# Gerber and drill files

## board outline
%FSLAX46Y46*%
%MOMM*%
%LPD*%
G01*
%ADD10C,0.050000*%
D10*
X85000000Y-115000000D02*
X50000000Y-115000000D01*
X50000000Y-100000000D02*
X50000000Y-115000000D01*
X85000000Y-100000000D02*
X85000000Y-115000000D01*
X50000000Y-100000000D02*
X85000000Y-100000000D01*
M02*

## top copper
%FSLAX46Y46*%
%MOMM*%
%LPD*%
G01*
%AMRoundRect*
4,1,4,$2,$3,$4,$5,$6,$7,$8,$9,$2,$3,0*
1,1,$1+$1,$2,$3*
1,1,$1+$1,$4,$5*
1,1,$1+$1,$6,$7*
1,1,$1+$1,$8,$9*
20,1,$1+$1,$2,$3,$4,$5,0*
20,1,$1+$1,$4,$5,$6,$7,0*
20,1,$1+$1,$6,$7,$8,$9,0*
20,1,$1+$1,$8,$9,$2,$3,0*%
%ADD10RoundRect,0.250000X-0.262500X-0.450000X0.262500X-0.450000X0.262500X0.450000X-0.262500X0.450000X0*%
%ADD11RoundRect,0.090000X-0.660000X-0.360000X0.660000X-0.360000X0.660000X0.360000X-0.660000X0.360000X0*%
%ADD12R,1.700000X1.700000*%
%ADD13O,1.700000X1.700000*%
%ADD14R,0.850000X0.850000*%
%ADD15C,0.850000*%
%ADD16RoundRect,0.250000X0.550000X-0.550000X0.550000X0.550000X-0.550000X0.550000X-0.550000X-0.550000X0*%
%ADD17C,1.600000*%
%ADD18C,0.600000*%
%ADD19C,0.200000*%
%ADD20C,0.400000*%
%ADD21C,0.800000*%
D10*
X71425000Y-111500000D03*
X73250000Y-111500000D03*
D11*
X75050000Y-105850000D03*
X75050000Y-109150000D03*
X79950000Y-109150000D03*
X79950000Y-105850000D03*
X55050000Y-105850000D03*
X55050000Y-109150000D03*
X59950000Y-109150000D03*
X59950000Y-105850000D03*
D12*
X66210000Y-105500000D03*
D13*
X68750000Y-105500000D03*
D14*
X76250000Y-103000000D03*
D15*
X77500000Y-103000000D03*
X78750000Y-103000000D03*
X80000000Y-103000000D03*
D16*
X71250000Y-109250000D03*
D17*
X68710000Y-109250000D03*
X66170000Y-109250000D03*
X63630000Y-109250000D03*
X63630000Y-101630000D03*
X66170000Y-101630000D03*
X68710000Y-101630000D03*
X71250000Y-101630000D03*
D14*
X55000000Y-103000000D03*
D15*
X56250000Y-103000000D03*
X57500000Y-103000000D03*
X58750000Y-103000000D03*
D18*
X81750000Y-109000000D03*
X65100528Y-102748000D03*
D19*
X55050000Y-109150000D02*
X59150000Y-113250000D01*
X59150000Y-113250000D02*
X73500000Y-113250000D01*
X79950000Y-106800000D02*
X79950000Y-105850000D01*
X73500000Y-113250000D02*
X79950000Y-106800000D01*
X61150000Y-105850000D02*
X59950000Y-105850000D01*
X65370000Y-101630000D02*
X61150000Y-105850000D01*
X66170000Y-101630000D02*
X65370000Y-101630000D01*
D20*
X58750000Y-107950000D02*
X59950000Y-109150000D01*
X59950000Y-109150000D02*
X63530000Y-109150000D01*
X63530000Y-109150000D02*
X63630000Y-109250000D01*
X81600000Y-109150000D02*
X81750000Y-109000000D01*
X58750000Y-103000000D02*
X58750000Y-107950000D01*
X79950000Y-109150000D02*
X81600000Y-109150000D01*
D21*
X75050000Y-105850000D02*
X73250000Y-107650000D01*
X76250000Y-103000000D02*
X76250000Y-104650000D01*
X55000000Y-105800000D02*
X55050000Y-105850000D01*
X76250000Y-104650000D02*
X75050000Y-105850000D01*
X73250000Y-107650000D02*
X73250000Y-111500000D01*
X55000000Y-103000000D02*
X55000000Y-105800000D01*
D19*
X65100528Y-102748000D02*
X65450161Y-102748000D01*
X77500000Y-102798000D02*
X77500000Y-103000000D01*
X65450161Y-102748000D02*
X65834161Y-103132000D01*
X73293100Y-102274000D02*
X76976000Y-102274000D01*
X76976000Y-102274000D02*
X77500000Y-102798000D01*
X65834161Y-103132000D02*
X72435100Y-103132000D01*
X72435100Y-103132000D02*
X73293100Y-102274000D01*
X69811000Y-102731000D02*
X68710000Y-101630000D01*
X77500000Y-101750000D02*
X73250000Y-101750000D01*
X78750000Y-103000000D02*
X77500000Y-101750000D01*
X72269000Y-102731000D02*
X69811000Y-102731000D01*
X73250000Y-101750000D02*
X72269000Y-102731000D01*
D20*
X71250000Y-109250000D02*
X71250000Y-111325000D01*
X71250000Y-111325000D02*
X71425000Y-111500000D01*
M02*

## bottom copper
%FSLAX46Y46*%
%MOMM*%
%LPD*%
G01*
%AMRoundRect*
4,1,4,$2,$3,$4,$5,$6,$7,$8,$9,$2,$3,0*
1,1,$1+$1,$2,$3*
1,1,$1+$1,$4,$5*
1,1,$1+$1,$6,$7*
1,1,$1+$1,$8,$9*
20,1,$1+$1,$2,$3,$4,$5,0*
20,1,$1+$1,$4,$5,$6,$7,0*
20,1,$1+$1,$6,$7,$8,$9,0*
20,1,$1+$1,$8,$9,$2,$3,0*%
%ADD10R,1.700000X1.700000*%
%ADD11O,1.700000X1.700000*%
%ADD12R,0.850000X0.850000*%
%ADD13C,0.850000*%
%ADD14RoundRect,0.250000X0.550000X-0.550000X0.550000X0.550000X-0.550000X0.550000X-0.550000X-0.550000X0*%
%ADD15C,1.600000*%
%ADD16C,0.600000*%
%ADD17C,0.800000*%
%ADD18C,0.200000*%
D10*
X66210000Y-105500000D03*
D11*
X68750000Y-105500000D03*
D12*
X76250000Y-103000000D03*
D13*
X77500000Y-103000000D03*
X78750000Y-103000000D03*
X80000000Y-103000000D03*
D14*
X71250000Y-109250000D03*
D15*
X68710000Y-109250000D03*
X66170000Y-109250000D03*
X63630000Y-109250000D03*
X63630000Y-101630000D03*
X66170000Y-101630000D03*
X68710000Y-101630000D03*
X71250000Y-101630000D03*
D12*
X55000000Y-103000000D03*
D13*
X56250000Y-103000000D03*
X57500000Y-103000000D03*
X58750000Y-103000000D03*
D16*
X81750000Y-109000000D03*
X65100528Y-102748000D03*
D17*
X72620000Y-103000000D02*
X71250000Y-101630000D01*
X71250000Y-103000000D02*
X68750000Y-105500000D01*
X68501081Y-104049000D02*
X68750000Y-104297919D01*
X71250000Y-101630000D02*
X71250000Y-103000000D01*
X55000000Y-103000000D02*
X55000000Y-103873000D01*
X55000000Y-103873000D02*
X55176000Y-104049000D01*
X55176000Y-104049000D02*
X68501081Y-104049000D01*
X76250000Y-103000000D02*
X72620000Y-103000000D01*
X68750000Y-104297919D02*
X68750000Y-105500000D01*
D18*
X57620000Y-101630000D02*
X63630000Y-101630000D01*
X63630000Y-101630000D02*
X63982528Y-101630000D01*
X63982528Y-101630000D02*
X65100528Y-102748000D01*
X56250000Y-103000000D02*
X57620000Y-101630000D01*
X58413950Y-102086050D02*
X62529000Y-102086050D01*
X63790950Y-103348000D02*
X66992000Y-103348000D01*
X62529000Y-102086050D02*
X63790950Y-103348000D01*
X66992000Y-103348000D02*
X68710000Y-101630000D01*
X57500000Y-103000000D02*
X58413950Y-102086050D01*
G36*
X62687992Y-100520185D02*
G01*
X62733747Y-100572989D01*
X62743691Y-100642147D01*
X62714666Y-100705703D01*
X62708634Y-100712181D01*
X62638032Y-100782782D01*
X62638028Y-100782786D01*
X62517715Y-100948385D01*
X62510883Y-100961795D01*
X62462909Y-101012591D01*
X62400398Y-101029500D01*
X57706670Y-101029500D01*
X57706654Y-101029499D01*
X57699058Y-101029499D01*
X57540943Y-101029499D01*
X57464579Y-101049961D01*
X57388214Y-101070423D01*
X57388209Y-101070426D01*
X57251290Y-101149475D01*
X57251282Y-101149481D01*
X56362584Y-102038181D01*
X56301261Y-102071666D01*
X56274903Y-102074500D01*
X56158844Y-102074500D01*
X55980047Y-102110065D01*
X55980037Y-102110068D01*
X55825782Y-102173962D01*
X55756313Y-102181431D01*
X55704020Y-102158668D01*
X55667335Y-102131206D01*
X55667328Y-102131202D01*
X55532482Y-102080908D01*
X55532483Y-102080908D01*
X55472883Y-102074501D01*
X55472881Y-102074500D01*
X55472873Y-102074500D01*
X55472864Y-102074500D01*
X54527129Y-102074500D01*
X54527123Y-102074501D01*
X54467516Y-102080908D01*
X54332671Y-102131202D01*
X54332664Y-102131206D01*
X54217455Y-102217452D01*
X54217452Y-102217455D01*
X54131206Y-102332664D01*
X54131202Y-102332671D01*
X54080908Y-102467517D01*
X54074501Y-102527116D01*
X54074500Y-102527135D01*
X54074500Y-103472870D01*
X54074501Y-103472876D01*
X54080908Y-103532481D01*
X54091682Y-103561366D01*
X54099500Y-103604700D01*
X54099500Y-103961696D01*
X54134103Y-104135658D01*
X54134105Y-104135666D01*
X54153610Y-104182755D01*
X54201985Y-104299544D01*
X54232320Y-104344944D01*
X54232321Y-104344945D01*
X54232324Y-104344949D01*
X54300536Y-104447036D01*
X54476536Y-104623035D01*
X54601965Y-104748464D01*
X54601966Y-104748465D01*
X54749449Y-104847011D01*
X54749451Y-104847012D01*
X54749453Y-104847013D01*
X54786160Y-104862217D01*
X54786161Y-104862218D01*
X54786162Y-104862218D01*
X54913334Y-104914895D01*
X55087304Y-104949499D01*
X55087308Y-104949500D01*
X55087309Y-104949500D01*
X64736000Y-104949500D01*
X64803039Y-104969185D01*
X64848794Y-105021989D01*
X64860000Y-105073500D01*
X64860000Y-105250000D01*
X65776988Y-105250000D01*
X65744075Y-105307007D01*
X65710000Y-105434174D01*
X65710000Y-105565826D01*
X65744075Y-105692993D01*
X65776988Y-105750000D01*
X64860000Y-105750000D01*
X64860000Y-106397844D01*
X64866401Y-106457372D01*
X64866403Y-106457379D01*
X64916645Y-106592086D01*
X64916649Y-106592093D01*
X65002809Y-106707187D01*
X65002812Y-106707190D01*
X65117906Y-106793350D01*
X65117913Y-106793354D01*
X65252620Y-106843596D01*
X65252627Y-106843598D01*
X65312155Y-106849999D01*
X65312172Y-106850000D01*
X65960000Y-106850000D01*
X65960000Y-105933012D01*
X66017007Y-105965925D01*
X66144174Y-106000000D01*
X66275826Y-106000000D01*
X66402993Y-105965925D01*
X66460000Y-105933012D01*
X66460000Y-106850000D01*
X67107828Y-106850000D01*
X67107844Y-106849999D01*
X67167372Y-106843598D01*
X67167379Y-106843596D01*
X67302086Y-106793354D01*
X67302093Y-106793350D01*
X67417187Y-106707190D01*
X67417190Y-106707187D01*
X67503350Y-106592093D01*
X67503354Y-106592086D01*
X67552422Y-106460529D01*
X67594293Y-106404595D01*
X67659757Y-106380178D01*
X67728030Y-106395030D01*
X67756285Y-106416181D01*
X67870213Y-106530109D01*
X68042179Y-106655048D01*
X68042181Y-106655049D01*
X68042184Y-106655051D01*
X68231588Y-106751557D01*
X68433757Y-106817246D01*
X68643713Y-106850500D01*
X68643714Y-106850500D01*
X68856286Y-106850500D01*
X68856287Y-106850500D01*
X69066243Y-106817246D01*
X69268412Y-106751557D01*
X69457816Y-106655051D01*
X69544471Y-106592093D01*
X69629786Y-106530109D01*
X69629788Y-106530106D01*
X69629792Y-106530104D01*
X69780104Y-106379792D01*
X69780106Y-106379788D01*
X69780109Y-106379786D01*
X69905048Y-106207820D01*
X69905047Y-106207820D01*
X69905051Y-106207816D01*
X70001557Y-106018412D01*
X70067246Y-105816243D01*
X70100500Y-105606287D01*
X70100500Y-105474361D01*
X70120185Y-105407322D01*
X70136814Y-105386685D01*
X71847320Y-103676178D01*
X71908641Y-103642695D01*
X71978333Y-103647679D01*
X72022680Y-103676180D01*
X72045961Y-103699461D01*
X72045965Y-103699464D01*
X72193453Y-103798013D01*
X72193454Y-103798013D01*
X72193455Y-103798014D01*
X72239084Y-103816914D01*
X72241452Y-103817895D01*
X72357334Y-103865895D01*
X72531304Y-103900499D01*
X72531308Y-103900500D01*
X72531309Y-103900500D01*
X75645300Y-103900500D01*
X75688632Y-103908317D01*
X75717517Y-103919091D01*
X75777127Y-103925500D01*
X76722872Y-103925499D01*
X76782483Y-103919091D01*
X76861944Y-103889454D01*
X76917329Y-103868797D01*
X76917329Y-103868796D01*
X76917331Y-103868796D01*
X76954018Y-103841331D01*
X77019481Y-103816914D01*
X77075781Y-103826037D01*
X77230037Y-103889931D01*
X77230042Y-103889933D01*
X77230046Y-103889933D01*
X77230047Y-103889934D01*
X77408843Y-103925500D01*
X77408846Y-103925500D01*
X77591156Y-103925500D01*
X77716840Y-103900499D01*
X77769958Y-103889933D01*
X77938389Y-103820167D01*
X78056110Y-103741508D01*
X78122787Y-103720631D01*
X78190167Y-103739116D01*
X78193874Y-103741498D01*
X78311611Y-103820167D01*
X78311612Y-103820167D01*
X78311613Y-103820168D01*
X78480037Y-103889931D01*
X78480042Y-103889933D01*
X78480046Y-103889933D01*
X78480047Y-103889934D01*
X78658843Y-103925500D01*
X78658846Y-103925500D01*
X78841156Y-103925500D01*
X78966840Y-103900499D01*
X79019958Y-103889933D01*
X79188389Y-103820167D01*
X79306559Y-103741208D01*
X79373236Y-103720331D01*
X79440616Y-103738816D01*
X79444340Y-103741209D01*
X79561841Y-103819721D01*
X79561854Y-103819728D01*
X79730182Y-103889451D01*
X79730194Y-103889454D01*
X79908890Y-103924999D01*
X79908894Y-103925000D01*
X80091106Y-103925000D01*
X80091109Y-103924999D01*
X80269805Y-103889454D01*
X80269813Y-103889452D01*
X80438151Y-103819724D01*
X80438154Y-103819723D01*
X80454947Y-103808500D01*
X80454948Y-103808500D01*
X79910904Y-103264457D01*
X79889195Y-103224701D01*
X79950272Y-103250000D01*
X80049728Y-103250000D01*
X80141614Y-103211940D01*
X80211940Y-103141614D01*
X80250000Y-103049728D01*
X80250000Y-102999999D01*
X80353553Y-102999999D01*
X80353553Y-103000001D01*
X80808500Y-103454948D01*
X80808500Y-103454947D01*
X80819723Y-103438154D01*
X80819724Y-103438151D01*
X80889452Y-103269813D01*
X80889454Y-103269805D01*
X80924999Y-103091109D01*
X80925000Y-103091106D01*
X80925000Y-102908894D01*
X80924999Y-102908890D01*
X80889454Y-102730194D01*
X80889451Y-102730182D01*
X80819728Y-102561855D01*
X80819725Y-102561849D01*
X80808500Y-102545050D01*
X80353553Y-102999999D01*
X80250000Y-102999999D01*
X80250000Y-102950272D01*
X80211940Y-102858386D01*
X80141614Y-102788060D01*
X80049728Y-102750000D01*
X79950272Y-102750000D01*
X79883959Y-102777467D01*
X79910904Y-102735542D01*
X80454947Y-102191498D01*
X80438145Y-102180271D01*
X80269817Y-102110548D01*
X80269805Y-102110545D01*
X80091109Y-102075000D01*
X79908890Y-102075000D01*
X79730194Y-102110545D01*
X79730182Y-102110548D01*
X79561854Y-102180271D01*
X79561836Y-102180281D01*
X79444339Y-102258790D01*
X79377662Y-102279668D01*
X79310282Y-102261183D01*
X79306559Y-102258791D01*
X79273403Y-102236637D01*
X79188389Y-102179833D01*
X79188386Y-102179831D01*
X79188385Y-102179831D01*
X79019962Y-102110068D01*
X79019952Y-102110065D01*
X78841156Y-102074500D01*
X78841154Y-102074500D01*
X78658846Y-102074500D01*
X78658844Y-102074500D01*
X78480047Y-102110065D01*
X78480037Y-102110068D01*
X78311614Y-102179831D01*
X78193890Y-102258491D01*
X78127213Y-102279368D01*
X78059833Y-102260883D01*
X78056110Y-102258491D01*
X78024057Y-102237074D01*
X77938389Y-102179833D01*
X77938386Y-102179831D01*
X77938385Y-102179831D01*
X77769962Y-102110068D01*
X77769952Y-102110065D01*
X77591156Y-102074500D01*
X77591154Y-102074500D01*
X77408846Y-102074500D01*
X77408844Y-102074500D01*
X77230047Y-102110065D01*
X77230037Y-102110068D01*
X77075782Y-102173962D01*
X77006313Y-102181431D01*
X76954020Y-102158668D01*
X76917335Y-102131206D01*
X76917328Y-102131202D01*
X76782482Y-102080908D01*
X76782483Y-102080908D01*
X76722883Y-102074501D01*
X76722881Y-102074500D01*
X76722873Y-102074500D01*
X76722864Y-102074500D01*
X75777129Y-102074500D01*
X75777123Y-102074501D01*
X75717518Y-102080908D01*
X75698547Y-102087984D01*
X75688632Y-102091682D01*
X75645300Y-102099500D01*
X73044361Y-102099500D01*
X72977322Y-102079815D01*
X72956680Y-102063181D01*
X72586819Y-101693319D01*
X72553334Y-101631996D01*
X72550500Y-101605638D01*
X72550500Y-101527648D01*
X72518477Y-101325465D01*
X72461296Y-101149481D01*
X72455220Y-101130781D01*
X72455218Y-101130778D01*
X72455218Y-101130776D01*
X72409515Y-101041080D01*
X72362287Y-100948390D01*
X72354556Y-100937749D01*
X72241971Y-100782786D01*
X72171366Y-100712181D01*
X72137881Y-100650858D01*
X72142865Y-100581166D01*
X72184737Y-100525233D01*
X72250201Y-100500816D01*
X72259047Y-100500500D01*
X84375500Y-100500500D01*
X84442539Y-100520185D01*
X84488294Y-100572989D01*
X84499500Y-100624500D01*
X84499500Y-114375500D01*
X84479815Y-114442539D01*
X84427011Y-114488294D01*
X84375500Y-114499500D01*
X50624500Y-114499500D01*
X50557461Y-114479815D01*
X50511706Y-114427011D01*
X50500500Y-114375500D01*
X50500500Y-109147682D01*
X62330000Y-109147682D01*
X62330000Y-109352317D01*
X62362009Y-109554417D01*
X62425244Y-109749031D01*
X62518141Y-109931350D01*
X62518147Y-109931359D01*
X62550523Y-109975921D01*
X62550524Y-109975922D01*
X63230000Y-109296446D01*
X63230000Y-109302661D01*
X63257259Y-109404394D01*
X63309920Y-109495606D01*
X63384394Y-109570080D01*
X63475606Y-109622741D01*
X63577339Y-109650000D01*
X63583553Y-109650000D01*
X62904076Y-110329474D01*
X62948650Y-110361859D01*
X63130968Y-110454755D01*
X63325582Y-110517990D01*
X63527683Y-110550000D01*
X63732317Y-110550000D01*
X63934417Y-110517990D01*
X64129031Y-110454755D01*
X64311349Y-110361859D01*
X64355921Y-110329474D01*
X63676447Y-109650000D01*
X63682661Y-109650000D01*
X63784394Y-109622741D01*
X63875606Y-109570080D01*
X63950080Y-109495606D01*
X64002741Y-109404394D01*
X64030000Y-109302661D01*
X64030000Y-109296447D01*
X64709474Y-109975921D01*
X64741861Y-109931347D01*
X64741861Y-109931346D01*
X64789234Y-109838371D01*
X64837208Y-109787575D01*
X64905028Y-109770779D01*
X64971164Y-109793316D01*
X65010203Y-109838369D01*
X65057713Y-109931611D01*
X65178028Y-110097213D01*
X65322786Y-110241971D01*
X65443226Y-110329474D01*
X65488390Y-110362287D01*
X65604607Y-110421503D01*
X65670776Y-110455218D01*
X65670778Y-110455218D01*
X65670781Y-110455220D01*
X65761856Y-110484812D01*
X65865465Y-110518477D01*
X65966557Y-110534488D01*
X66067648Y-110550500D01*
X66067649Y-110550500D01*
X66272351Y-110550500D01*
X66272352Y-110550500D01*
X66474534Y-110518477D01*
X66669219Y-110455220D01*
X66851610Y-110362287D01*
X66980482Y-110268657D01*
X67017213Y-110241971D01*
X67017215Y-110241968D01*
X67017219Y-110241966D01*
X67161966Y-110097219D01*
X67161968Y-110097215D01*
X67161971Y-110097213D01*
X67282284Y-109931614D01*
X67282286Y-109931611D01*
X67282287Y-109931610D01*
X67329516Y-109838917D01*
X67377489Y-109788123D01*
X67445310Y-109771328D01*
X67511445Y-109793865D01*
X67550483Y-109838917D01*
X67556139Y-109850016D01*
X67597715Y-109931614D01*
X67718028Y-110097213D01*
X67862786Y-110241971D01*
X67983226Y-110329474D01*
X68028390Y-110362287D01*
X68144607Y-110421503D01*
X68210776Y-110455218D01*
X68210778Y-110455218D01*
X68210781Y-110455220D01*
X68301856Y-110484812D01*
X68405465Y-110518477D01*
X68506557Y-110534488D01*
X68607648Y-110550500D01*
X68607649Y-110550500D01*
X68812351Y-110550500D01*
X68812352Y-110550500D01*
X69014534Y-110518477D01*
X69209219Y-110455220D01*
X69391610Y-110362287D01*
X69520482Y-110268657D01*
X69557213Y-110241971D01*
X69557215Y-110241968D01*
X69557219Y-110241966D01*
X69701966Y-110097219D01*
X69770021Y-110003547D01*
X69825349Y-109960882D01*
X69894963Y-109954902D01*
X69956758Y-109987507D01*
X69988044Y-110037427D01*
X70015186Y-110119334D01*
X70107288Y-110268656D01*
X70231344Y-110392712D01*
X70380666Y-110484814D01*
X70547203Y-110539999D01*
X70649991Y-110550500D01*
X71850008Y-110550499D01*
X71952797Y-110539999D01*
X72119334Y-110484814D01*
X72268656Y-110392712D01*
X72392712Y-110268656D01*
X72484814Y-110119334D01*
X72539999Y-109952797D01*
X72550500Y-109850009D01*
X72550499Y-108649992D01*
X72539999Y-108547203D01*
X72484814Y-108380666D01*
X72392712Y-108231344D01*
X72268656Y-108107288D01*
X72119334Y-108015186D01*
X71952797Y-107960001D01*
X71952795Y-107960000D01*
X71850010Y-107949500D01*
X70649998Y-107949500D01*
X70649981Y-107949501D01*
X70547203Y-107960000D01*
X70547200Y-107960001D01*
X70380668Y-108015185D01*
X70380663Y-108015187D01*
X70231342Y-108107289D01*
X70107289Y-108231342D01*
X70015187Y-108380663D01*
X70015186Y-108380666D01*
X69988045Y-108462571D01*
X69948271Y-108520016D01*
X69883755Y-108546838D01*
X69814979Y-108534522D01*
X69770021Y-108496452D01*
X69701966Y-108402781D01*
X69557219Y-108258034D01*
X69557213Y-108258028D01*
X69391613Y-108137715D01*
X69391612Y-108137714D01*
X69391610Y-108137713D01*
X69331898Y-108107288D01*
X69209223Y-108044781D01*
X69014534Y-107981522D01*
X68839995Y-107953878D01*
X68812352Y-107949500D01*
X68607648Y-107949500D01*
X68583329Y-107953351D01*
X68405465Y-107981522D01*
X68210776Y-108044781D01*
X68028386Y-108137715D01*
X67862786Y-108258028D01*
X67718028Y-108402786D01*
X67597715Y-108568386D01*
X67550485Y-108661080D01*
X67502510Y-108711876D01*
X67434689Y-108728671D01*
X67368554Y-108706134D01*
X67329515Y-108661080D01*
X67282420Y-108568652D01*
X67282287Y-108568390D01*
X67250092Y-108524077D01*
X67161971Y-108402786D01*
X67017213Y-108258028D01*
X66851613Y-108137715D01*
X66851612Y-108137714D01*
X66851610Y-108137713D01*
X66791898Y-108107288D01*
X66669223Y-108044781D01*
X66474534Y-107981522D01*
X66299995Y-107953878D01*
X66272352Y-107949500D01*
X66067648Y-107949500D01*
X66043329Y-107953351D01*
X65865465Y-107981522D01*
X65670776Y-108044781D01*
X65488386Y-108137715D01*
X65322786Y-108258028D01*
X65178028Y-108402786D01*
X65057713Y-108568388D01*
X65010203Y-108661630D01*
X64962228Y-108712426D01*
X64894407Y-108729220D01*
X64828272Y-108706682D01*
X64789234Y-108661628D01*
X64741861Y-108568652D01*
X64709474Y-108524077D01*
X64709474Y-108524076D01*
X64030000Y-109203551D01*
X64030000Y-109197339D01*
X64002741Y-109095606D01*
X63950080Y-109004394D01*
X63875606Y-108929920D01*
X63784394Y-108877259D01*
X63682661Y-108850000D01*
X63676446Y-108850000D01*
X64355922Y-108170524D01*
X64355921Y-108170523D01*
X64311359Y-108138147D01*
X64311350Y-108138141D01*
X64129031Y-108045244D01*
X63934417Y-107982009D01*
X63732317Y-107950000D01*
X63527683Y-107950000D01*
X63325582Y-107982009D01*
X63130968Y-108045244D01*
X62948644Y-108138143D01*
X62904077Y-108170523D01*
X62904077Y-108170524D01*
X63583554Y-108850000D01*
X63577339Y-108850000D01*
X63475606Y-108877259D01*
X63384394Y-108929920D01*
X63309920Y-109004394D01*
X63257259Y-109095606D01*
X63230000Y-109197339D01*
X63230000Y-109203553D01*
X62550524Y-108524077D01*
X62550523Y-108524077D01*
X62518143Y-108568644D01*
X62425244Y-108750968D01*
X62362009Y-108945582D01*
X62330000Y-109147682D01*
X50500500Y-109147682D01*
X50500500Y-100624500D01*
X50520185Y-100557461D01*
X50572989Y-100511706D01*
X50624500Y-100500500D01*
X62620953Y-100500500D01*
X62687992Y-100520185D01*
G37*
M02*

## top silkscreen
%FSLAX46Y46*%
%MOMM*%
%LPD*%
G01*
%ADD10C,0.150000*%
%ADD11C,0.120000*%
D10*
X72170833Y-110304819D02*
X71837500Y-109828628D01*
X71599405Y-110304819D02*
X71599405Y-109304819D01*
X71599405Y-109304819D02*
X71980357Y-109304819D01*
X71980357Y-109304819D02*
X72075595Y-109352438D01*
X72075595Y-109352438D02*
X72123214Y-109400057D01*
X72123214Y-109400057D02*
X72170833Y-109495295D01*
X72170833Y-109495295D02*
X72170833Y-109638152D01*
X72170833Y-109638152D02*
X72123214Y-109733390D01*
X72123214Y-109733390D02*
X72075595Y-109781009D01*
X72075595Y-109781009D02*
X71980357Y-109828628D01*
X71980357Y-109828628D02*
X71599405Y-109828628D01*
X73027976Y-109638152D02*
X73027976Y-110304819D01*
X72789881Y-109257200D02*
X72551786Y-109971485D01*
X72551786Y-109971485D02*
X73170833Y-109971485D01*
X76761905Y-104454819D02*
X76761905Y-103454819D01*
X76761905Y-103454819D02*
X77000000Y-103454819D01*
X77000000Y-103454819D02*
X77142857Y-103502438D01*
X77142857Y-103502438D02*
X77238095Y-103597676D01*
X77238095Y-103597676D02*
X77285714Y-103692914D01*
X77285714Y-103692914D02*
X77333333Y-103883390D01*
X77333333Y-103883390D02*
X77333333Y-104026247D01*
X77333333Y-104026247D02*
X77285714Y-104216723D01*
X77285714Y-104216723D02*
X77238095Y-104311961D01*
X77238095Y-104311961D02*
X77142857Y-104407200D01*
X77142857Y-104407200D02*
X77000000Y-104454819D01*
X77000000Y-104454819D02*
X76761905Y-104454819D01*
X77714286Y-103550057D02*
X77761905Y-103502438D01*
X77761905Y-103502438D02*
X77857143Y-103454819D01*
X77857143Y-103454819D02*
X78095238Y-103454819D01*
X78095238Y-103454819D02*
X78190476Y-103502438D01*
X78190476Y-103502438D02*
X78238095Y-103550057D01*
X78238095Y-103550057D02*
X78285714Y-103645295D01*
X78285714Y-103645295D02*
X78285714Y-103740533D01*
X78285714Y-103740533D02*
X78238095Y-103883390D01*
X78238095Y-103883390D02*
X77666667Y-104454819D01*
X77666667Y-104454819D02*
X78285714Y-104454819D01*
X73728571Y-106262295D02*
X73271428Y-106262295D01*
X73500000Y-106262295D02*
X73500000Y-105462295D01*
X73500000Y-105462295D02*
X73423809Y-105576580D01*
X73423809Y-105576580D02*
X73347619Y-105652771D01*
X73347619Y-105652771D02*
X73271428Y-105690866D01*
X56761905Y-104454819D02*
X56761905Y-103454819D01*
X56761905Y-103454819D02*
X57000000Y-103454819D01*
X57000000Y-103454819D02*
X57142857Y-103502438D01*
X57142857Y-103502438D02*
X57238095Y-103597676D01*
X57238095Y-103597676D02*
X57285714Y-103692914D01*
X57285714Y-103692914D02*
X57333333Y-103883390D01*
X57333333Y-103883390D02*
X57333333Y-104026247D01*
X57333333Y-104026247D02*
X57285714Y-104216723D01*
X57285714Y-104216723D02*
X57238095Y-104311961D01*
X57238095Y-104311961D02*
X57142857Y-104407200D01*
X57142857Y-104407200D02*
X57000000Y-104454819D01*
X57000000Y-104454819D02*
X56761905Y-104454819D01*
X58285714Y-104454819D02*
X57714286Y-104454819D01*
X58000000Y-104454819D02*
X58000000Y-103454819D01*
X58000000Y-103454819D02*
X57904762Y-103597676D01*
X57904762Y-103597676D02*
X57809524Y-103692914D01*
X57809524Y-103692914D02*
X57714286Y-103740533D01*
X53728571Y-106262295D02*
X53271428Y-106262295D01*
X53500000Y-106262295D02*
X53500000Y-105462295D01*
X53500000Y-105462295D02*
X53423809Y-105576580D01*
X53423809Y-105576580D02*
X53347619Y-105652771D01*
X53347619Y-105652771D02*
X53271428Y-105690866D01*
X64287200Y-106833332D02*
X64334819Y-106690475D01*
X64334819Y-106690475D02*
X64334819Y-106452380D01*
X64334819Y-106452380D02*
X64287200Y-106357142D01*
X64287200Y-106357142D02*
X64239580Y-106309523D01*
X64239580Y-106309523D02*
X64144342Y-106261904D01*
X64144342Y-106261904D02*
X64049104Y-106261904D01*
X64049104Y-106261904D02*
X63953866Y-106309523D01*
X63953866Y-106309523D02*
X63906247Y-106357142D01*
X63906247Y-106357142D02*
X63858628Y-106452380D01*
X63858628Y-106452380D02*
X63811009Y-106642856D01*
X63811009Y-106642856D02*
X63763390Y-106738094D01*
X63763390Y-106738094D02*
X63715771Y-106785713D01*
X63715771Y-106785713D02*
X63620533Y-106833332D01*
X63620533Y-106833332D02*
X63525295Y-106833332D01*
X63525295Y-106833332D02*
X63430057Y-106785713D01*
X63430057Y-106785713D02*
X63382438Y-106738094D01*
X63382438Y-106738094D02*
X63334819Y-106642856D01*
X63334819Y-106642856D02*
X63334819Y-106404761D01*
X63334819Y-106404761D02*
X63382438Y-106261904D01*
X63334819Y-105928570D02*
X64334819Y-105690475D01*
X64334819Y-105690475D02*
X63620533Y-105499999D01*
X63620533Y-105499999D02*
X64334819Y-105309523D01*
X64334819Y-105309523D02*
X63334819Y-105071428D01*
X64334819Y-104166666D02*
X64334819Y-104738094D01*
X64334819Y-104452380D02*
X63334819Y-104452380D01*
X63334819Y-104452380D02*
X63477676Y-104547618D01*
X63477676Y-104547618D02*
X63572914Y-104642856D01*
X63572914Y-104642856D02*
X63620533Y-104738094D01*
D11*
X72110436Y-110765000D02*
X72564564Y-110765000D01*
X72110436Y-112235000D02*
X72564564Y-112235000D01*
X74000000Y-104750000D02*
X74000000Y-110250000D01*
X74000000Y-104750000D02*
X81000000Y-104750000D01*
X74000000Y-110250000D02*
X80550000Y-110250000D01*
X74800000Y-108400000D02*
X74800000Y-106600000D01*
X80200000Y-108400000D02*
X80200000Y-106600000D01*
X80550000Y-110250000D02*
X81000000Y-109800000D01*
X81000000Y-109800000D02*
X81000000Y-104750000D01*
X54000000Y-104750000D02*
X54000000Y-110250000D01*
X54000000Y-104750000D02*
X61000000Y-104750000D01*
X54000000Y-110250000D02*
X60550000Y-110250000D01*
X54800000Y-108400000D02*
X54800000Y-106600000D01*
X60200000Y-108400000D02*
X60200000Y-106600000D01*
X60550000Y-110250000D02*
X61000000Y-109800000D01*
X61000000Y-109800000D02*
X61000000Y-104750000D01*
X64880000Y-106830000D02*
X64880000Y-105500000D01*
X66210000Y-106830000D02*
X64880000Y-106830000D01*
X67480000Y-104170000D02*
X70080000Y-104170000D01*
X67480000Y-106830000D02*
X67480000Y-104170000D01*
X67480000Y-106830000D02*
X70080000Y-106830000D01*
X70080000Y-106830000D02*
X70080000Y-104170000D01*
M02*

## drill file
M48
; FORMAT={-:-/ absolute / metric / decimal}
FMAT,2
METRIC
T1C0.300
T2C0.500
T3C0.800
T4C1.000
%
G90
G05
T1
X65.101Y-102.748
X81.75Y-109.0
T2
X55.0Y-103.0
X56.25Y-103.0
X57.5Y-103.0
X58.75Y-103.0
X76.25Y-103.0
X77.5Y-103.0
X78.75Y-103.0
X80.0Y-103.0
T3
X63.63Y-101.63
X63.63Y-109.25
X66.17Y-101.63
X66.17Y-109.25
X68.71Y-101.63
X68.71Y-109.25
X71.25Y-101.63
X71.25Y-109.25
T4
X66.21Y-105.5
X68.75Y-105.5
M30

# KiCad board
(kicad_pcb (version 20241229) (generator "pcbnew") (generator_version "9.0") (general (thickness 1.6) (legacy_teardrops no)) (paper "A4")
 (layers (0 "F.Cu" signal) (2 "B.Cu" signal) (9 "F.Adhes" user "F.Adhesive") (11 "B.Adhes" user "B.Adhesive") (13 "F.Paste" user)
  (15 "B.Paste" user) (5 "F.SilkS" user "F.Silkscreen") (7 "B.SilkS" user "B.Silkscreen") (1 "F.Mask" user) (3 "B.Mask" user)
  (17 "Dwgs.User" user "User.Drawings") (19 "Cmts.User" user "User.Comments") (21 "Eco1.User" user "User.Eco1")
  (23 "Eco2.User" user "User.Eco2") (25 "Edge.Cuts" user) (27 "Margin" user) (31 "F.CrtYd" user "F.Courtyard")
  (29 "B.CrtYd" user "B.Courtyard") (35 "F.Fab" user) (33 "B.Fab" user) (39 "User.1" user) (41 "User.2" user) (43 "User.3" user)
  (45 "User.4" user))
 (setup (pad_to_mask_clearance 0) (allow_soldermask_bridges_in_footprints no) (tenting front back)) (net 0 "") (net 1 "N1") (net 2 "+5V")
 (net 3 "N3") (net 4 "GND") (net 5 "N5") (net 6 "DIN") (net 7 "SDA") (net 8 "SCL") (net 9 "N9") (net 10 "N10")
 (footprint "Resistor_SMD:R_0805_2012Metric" (layer "F.Cu") (at 72.3375 111.5)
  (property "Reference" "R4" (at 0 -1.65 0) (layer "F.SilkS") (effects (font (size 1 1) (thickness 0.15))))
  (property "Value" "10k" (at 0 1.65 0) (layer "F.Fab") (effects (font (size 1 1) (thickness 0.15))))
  (fp_line (start -0.227064 -0.735) (end 0.227064 -0.735) (stroke (width 0.12) (type solid)) (layer "F.SilkS"))
  (fp_line (start -0.227064 0.735) (end 0.227064 0.735) (stroke (width 0.12) (type solid)) (layer "F.SilkS"))
  (pad "1" smd roundrect (at -0.9125 0) (size 1.025 1.4) (layers "F.Cu" "F.Mask" "F.Paste") (roundrect_rratio 0.243902) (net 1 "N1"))
  (pad "2" smd roundrect (at 0.9125 0) (size 1.025 1.4) (layers "F.Cu" "F.Mask" "F.Paste") (roundrect_rratio 0.243902) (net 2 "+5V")))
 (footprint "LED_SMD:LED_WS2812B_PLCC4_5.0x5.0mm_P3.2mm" (layer "F.Cu") (at 77.5 107.5)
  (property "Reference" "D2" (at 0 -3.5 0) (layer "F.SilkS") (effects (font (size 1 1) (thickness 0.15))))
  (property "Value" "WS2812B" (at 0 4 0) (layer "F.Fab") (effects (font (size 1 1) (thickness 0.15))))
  (fp_line (start -3.5 -2.75) (end -3.5 2.75) (stroke (width 0.12) (type default)) (layer "F.SilkS"))
  (fp_line (start -3.5 -2.75) (end 3.5 -2.75) (stroke (width 0.12) (type solid)) (layer "F.SilkS"))
  (fp_line (start -3.5 2.75) (end 3.05 2.75) (stroke (width 0.12) (type solid)) (layer "F.SilkS"))
  (fp_line (start -2.7 0.9) (end -2.7 -0.9) (stroke (width 0.12) (type default)) (layer "F.SilkS"))
  (fp_line (start 2.7 0.9) (end 2.7 -0.9) (stroke (width 0.12) (type default)) (layer "F.SilkS"))
  (fp_line (start 3.05 2.75) (end 3.5 2.3) (stroke (width 0.12) (type default)) (layer "F.SilkS"))
  (fp_line (start 3.5 2.3) (end 3.5 -2.75) (stroke (width 0.12) (type default)) (layer "F.SilkS"))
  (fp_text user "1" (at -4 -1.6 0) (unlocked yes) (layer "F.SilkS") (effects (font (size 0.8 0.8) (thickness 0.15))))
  (pad "1" smd roundrect (at -2.45 -1.65) (size 1.5 0.9) (layers "F.Cu" "F.Mask" "F.Paste") (roundrect_rratio 0.1) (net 2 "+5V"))
  (pad "2" smd roundrect (at -2.45 1.65) (size 1.5 0.9) (layers "F.Cu" "F.Mask" "F.Paste") (roundrect_rratio 0.1) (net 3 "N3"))
  (pad "3" smd roundrect (at 2.45 1.65) (size 1.5 0.9) (layers "F.Cu" "F.Mask" "F.Paste") (roundrect_rratio 0.1) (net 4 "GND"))
  (pad "4" smd roundrect (at 2.45 -1.65) (size 1.5 0.9) (layers "F.Cu" "F.Mask" "F.Paste") (roundrect_rratio 0.1) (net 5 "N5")))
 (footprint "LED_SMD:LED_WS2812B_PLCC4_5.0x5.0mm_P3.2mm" (layer "F.Cu") (at 57.5 107.5)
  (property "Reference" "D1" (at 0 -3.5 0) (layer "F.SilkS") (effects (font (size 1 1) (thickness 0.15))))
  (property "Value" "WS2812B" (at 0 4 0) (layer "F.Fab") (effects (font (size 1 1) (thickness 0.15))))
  (fp_line (start -3.5 -2.75) (end -3.5 2.75) (stroke (width 0.12) (type default)) (layer "F.SilkS"))
  (fp_line (start -3.5 -2.75) (end 3.5 -2.75) (stroke (width 0.12) (type solid)) (layer "F.SilkS"))
  (fp_line (start -3.5 2.75) (end 3.05 2.75) (stroke (width 0.12) (type solid)) (layer "F.SilkS"))
  (fp_line (start -2.7 0.9) (end -2.7 -0.9) (stroke (width 0.12) (type default)) (layer "F.SilkS"))
  (fp_line (start 2.7 0.9) (end 2.7 -0.9) (stroke (width 0.12) (type default)) (layer "F.SilkS"))
  (fp_line (start 3.05 2.75) (end 3.5 2.3) (stroke (width 0.12) (type default)) (layer "F.SilkS"))
  (fp_line (start 3.5 2.3) (end 3.5 -2.75) (stroke (width 0.12) (type default)) (layer "F.SilkS"))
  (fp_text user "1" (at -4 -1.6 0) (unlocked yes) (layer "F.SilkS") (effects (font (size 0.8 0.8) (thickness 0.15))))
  (pad "1" smd roundrect (at -2.45 -1.65) (size 1.5 0.9) (layers "F.Cu" "F.Mask" "F.Paste") (roundrect_rratio 0.1) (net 2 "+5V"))
  (pad "2" smd roundrect (at -2.45 1.65) (size 1.5 0.9) (layers "F.Cu" "F.Mask" "F.Paste") (roundrect_rratio 0.1) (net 5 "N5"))
  (pad "3" smd roundrect (at 2.45 1.65) (size 1.5 0.9) (layers "F.Cu" "F.Mask" "F.Paste") (roundrect_rratio 0.1) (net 4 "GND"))
  (pad "4" smd roundrect (at 2.45 -1.65) (size 1.5 0.9) (layers "F.Cu" "F.Mask" "F.Paste") (roundrect_rratio 0.1) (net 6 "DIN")))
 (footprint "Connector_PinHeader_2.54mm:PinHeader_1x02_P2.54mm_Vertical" (layer "F.Cu") (at 66.21 105.5 90)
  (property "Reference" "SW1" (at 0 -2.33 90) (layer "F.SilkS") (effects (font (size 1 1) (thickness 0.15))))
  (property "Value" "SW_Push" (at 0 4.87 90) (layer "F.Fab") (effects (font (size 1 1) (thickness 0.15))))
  (fp_line (start -1.33 -1.33) (end 0 -1.33) (stroke (width 0.12) (type solid)) (layer "F.SilkS"))
  (fp_line (start -1.33 0) (end -1.33 -1.33) (stroke (width 0.12) (type solid)) (layer "F.SilkS"))
  (fp_line (start 1.33 1.27) (end 1.33 3.87) (stroke (width 0.12) (type solid)) (layer "F.SilkS"))
  (fp_line (start -1.33 1.27) (end 1.33 1.27) (stroke (width 0.12) (type solid)) (layer "F.SilkS"))
  (fp_line (start -1.33 1.27) (end -1.33 3.87) (stroke (width 0.12) (type solid)) (layer "F.SilkS"))
  (fp_line (start -1.33 3.87) (end 1.33 3.87) (stroke (width 0.12) (type solid)) (layer "F.SilkS"))
  (pad "1" thru_hole rect (at 0 0 90) (size 1.7 1.7) (drill 1) (layers "*.Cu" "*.Mask") (remove_unused_layers no) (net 4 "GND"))
  (pad "2" thru_hole oval (at 0 2.54 90) (size 1.7 1.7) (drill 1) (layers "*.Cu" "*.Mask") (remove_unused_layers no) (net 2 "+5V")))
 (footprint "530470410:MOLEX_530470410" (layer "B.Cu") (at 76.25 103 180)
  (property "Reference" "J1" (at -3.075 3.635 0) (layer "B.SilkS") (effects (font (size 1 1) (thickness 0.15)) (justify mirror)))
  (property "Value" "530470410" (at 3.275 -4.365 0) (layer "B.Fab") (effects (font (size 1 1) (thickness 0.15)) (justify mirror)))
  (pad "1" thru_hole rect (at 0 0 180) (size 0.85 0.85) (drill 0.5) (layers "*.Cu") (remove_unused_layers no) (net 2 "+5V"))
  (pad "2" thru_hole circle (at -1.25 0 180) (size 0.85 0.85) (drill 0.5) (layers "*.Cu") (remove_unused_layers no) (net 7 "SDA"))
  (pad "3" thru_hole circle (at -2.5 0 180) (size 0.85 0.85) (drill 0.5) (layers "*.Cu") (remove_unused_layers no) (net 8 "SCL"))
  (pad "4" thru_hole circle (at -3.75 0 180) (size 0.85 0.85) (drill 0.5) (layers "*.Cu") (remove_unused_layers no) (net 4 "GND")))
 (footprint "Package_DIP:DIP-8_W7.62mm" (layer "B.Cu") (at 71.25 109.25 90)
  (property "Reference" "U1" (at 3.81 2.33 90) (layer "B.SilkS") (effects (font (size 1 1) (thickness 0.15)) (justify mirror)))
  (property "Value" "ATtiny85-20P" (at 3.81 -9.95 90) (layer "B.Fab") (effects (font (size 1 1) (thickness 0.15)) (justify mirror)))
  (pad "1" thru_hole roundrect (at 0 0 90) (size 1.6 1.6) (drill 0.8) (layers "*.Cu" "*.Mask") (remove_unused_layers no)
   (roundrect_rratio 0.15625) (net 1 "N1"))
  (pad "2" thru_hole circle (at 0 -2.54 90) (size 1.6 1.6) (drill 0.8) (layers "*.Cu" "*.Mask") (remove_unused_layers no) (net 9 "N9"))
  (pad "3" thru_hole circle (at 0 -5.08 90) (size 1.6 1.6) (drill 0.8) (layers "*.Cu" "*.Mask") (remove_unused_layers no) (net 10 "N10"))
  (pad "4" thru_hole circle (at 0 -7.62 90) (size 1.6 1.6) (drill 0.8) (layers "*.Cu" "*.Mask") (remove_unused_layers no) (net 4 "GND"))
  (pad "5" thru_hole circle (at 7.62 -7.62 90) (size 1.6 1.6) (drill 0.8) (layers "*.Cu" "*.Mask") (remove_unused_layers no) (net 7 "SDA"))
  (pad "6" thru_hole circle (at 7.62 -5.08 90) (size 1.6 1.6) (drill 0.8) (layers "*.Cu" "*.Mask") (remove_unused_layers no) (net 6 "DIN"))
  (pad "7" thru_hole circle (at 7.62 -2.54 90) (size 1.6 1.6) (drill 0.8) (layers "*.Cu" "*.Mask") (remove_unused_layers no) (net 8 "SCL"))
  (pad "8" thru_hole circle (at 7.62 0 90) (size 1.6 1.6) (drill 0.8) (layers "*.Cu" "*.Mask") (remove_unused_layers no) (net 2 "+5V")))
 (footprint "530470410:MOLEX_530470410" (layer "B.Cu") (at 55 103 180)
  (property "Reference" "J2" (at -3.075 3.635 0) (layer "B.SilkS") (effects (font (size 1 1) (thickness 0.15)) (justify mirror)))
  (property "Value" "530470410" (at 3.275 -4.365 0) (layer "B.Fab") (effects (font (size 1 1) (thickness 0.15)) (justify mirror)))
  (pad "1" thru_hole rect (at 0 0 180) (size 0.85 0.85) (drill 0.5) (layers "*.Cu") (remove_unused_layers no) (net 2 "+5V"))
  (pad "2" thru_hole circle (at -1.25 0 180) (size 0.85 0.85) (drill 0.5) (layers "*.Cu") (remove_unused_layers no) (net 7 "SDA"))
  (pad "3" thru_hole circle (at -2.5 0 180) (size 0.85 0.85) (drill 0.5) (layers "*.Cu") (remove_unused_layers no) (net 8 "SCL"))
  (pad "4" thru_hole circle (at -3.75 0 180) (size 0.85 0.85) (drill 0.5) (layers "*.Cu") (remove_unused_layers no) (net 4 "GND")))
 (gr_line (start 85 115) (end 50 115) (stroke (width 0.05) (type default)) (layer "Edge.Cuts"))
 (gr_line (start 50 100) (end 50 115) (stroke (width 0.05) (type default)) (layer "Edge.Cuts"))
 (gr_line (start 85 100) (end 85 115) (stroke (width 0.05) (type default)) (layer "Edge.Cuts"))
 (gr_line (start 50 100) (end 85 100) (stroke (width 0.05) (type default)) (layer "Edge.Cuts"))
 (segment (start 55.05 109.15) (end 59.15 113.25) (width 0.2) (layer "F.Cu") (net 5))
 (segment (start 59.15 113.25) (end 73.5 113.25) (width 0.2) (layer "F.Cu") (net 5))
 (segment (start 79.95 106.8) (end 79.95 105.85) (width 0.2) (layer "F.Cu") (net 5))
 (segment (start 73.5 113.25) (end 79.95 106.8) (width 0.2) (layer "F.Cu") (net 5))
 (segment (start 61.15 105.85) (end 59.95 105.85) (width 0.2) (layer "F.Cu") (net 6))
 (segment (start 65.37 101.63) (end 61.15 105.85) (width 0.2) (layer "F.Cu") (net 6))
 (segment (start 66.17 101.63) (end 65.37 101.63) (width 0.2) (layer "F.Cu") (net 6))
 (segment (start 58.75 107.95) (end 59.95 109.15) (width 0.4) (layer "F.Cu") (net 4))
 (segment (start 59.95 109.15) (end 63.53 109.15) (width 0.4) (layer "F.Cu") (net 4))
 (segment (start 63.53 109.15) (end 63.63 109.25) (width 0.4) (layer "F.Cu") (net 4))
 (segment (start 81.6 109.15) (end 81.75 109) (width 0.4) (layer "F.Cu") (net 4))
 (segment (start 58.75 103) (end 58.75 107.95) (width 0.4) (layer "F.Cu") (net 4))
 (segment (start 79.95 109.15) (end 81.6 109.15) (width 0.4) (layer "F.Cu") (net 4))
 (via (at 81.75 109) (size 0.6) (drill 0.3) (layers "F.Cu" "B.Cu") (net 4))
 (segment (start 75.05 105.85) (end 73.25 107.65) (width 0.8) (layer "F.Cu") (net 2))
 (segment (start 76.25 103) (end 76.25 104.65) (width 0.8) (layer "F.Cu") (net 2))
 (segment (start 55 105.8) (end 55.05 105.85) (width 0.8) (layer "F.Cu") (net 2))
 (segment (start 76.25 104.65) (end 75.05 105.85) (width 0.8) (layer "F.Cu") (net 2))
 (segment (start 73.25 107.65) (end 73.25 111.5) (width 0.8) (layer "F.Cu") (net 2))
 (segment (start 55 103) (end 55 105.8) (width 0.8) (layer "F.Cu") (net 2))
 (segment (start 72.62 103) (end 71.25 101.63) (width 0.8) (layer "B.Cu") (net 2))
 (segment (start 71.25 103) (end 68.75 105.5) (width 0.8) (layer "B.Cu") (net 2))
 (segment (start 68.501081 104.049) (end 68.75 104.297919) (width 0.8) (layer "B.Cu") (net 2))
 (segment (start 71.25 101.63) (end 71.25 103) (width 0.8) (layer "B.Cu") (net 2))
 (segment (start 55 103) (end 55 103.873) (width 0.8) (layer "B.Cu") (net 2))
 (segment (start 55 103.873) (end 55.176 104.049) (width 0.8) (layer "B.Cu") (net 2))
 (segment (start 55.176 104.049) (end 68.501081 104.049) (width 0.8) (layer "B.Cu") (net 2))
 (segment (start 76.25 103) (end 72.62 103) (width 0.8) (layer "B.Cu") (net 2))
 (segment (start 68.75 104.297919) (end 68.75 105.5) (width 0.8) (layer "B.Cu") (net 2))
 (segment (start 65.100528 102.748) (end 65.450161 102.748) (width 0.2) (layer "F.Cu") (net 7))
 (segment (start 77.5 102.798) (end 77.5 103) (width 0.2) (layer "F.Cu") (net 7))
 (segment (start 65.450161 102.748) (end 65.834161 103.132) (width 0.2) (layer "F.Cu") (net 7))
 (segment (start 73.2931 102.274) (end 76.976 102.274) (width 0.2) (layer "F.Cu") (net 7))
 (segment (start 76.976 102.274) (end 77.5 102.798) (width 0.2) (layer "F.Cu") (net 7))
 (segment (start 65.834161 103.132) (end 72.4351 103.132) (width 0.2) (layer "F.Cu") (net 7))
 (segment (start 72.4351 103.132) (end 73.2931 102.274) (width 0.2) (layer "F.Cu") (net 7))
 (via (at 65.100528 102.748) (size 0.6) (drill 0.3) (layers "F.Cu" "B.Cu") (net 7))
 (segment (start 57.62 101.63) (end 63.63 101.63) (width 0.2) (layer "B.Cu") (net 7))
 (segment (start 63.63 101.63) (end 63.982528 101.63) (width 0.2) (layer "B.Cu") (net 7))
 (segment (start 63.982528 101.63) (end 65.100528 102.748) (width 0.2) (layer "B.Cu") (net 7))
 (segment (start 56.25 103) (end 57.62 101.63) (width 0.2) (layer "B.Cu") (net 7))
 (segment (start 69.811 102.731) (end 68.71 101.63) (width 0.2) (layer "F.Cu") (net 8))
 (segment (start 77.5 101.75) (end 73.25 101.75) (width 0.2) (layer "F.Cu") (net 8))
 (segment (start 78.75 103) (end 77.5 101.75) (width 0.2) (layer "F.Cu") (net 8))
 (segment (start 72.269 102.731) (end 69.811 102.731) (width 0.2) (layer "F.Cu") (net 8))
 (segment (start 73.25 101.75) (end 72.269 102.731) (width 0.2) (layer "F.Cu") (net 8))
 (segment (start 58.41395 102.08605) (end 62.529 102.08605) (width 0.2) (layer "B.Cu") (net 8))
 (segment (start 63.79095 103.348) (end 66.992 103.348) (width 0.2) (layer "B.Cu") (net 8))
 (segment (start 62.529 102.08605) (end 63.79095 103.348) (width 0.2) (layer "B.Cu") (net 8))
 (segment (start 66.992 103.348) (end 68.71 101.63) (width 0.2) (layer "B.Cu") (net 8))
 (segment (start 57.5 103) (end 58.41395 102.08605) (width 0.2) (layer "B.Cu") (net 8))
 (segment (start 71.25 109.25) (end 71.25 111.325) (width 0.4) (layer "F.Cu") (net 1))
 (segment (start 71.25 111.325) (end 71.425 111.5) (width 0.4) (layer "F.Cu") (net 1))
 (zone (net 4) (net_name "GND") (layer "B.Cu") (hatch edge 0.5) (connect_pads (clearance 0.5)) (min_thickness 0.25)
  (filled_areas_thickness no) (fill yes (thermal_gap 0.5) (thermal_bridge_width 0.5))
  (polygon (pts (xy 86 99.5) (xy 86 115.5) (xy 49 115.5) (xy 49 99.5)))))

